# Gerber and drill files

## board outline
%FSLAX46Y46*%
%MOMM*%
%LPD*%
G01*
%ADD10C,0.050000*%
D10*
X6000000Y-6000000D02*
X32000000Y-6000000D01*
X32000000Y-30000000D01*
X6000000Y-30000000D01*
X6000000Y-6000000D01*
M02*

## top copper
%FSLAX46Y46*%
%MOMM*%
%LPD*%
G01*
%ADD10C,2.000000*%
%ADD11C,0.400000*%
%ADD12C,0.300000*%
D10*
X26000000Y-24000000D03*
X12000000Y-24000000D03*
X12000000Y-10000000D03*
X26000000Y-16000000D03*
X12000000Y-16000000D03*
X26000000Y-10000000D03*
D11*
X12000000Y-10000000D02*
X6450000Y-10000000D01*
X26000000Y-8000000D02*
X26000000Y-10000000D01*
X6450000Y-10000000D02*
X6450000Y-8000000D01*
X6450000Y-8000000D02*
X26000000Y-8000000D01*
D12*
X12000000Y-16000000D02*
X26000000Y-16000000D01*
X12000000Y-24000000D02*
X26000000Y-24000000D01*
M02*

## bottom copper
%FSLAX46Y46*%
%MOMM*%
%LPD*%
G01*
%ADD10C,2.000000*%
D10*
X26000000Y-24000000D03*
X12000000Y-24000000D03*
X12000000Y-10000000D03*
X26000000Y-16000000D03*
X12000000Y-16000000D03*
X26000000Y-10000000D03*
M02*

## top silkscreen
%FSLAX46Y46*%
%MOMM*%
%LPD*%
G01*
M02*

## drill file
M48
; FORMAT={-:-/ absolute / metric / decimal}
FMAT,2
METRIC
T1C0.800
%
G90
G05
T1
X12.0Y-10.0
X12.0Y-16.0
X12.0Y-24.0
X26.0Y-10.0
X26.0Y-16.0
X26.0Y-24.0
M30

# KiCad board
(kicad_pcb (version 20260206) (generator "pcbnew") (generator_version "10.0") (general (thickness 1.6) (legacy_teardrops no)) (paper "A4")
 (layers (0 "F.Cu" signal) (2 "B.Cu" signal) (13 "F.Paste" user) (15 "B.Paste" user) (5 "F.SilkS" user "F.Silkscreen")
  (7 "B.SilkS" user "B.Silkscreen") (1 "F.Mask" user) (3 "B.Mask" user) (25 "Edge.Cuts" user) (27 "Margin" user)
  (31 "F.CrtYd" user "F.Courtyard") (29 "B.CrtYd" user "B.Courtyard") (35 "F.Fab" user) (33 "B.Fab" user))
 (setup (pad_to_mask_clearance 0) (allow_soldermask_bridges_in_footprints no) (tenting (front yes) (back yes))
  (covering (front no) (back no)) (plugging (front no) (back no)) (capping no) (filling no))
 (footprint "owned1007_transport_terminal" (layer "F.Cu") (at 26 24)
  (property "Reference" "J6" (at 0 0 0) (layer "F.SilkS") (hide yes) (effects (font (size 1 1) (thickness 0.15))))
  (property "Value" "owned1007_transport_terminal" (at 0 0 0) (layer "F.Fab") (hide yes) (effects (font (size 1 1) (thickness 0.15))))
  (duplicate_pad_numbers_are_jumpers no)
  (pad "1" thru_hole circle (at 0 0) (size 2 2) (drill 0.8) (layers "*.Cu" "*.Mask") (remove_unused_layers no) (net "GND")))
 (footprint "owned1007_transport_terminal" (layer "F.Cu") (at 12 24)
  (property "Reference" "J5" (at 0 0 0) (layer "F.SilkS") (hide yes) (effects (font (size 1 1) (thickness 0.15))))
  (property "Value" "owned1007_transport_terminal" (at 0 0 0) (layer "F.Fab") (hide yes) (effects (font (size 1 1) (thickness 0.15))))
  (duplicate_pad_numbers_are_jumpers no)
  (pad "1" thru_hole circle (at 0 0) (size 2 2) (drill 0.8) (layers "*.Cu" "*.Mask") (remove_unused_layers no) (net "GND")))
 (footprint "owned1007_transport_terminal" (layer "F.Cu") (at 12 10)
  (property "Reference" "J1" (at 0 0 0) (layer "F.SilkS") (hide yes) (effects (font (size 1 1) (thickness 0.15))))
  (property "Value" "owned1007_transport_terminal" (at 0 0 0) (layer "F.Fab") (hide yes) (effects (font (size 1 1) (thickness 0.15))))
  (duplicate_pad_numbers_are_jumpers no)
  (pad "1" thru_hole circle (at 0 0) (size 2 2) (drill 0.8) (layers "*.Cu" "*.Mask") (remove_unused_layers no) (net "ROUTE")))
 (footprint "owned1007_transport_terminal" (layer "F.Cu") (at 26 16)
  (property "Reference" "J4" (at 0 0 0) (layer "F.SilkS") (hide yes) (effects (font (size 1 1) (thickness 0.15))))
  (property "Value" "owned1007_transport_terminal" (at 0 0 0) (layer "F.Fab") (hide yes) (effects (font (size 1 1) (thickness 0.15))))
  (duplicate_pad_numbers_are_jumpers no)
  (pad "1" thru_hole circle (at 0 0) (size 2 2) (drill 0.8) (layers "*.Cu" "*.Mask") (remove_unused_layers no) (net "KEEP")))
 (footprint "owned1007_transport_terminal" (layer "F.Cu") (at 12 16)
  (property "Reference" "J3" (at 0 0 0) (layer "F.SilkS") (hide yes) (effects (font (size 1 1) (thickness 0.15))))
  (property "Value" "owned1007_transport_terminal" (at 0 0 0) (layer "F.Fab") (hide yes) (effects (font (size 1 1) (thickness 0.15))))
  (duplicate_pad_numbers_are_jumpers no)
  (pad "1" thru_hole circle (at 0 0) (size 2 2) (drill 0.8) (layers "*.Cu" "*.Mask") (remove_unused_layers no) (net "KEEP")))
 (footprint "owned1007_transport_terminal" (layer "F.Cu") (at 26 10)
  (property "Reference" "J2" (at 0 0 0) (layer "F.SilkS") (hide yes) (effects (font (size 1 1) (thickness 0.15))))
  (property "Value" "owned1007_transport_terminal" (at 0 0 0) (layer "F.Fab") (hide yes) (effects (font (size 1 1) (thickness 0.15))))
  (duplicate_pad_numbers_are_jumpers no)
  (pad "1" thru_hole circle (at 0 0) (size 2 2) (drill 0.8) (layers "*.Cu" "*.Mask") (remove_unused_layers no) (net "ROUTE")))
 (gr_rect (start 6 6) (end 32 30) (stroke (width 0.05) (type default)) (fill no) (layer "Edge.Cuts"))
 (segment (start 12 10) (end 6.45 10) (width 0.4) (layer "F.Cu") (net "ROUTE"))
 (segment (start 26 8) (end 26 10) (width 0.4) (layer "F.Cu") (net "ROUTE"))
 (segment (start 6.45 10) (end 6.45 8) (width 0.4) (layer "F.Cu") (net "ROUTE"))
 (segment (start 6.45 8) (end 26 8) (width 0.4) (layer "F.Cu") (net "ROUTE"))
 (segment (start 12 16) (end 26 16) (width 0.3) (locked yes) (layer "F.Cu") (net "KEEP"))
 (segment (start 12 24) (end 26 24) (width 0.3) (layer "F.Cu") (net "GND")))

